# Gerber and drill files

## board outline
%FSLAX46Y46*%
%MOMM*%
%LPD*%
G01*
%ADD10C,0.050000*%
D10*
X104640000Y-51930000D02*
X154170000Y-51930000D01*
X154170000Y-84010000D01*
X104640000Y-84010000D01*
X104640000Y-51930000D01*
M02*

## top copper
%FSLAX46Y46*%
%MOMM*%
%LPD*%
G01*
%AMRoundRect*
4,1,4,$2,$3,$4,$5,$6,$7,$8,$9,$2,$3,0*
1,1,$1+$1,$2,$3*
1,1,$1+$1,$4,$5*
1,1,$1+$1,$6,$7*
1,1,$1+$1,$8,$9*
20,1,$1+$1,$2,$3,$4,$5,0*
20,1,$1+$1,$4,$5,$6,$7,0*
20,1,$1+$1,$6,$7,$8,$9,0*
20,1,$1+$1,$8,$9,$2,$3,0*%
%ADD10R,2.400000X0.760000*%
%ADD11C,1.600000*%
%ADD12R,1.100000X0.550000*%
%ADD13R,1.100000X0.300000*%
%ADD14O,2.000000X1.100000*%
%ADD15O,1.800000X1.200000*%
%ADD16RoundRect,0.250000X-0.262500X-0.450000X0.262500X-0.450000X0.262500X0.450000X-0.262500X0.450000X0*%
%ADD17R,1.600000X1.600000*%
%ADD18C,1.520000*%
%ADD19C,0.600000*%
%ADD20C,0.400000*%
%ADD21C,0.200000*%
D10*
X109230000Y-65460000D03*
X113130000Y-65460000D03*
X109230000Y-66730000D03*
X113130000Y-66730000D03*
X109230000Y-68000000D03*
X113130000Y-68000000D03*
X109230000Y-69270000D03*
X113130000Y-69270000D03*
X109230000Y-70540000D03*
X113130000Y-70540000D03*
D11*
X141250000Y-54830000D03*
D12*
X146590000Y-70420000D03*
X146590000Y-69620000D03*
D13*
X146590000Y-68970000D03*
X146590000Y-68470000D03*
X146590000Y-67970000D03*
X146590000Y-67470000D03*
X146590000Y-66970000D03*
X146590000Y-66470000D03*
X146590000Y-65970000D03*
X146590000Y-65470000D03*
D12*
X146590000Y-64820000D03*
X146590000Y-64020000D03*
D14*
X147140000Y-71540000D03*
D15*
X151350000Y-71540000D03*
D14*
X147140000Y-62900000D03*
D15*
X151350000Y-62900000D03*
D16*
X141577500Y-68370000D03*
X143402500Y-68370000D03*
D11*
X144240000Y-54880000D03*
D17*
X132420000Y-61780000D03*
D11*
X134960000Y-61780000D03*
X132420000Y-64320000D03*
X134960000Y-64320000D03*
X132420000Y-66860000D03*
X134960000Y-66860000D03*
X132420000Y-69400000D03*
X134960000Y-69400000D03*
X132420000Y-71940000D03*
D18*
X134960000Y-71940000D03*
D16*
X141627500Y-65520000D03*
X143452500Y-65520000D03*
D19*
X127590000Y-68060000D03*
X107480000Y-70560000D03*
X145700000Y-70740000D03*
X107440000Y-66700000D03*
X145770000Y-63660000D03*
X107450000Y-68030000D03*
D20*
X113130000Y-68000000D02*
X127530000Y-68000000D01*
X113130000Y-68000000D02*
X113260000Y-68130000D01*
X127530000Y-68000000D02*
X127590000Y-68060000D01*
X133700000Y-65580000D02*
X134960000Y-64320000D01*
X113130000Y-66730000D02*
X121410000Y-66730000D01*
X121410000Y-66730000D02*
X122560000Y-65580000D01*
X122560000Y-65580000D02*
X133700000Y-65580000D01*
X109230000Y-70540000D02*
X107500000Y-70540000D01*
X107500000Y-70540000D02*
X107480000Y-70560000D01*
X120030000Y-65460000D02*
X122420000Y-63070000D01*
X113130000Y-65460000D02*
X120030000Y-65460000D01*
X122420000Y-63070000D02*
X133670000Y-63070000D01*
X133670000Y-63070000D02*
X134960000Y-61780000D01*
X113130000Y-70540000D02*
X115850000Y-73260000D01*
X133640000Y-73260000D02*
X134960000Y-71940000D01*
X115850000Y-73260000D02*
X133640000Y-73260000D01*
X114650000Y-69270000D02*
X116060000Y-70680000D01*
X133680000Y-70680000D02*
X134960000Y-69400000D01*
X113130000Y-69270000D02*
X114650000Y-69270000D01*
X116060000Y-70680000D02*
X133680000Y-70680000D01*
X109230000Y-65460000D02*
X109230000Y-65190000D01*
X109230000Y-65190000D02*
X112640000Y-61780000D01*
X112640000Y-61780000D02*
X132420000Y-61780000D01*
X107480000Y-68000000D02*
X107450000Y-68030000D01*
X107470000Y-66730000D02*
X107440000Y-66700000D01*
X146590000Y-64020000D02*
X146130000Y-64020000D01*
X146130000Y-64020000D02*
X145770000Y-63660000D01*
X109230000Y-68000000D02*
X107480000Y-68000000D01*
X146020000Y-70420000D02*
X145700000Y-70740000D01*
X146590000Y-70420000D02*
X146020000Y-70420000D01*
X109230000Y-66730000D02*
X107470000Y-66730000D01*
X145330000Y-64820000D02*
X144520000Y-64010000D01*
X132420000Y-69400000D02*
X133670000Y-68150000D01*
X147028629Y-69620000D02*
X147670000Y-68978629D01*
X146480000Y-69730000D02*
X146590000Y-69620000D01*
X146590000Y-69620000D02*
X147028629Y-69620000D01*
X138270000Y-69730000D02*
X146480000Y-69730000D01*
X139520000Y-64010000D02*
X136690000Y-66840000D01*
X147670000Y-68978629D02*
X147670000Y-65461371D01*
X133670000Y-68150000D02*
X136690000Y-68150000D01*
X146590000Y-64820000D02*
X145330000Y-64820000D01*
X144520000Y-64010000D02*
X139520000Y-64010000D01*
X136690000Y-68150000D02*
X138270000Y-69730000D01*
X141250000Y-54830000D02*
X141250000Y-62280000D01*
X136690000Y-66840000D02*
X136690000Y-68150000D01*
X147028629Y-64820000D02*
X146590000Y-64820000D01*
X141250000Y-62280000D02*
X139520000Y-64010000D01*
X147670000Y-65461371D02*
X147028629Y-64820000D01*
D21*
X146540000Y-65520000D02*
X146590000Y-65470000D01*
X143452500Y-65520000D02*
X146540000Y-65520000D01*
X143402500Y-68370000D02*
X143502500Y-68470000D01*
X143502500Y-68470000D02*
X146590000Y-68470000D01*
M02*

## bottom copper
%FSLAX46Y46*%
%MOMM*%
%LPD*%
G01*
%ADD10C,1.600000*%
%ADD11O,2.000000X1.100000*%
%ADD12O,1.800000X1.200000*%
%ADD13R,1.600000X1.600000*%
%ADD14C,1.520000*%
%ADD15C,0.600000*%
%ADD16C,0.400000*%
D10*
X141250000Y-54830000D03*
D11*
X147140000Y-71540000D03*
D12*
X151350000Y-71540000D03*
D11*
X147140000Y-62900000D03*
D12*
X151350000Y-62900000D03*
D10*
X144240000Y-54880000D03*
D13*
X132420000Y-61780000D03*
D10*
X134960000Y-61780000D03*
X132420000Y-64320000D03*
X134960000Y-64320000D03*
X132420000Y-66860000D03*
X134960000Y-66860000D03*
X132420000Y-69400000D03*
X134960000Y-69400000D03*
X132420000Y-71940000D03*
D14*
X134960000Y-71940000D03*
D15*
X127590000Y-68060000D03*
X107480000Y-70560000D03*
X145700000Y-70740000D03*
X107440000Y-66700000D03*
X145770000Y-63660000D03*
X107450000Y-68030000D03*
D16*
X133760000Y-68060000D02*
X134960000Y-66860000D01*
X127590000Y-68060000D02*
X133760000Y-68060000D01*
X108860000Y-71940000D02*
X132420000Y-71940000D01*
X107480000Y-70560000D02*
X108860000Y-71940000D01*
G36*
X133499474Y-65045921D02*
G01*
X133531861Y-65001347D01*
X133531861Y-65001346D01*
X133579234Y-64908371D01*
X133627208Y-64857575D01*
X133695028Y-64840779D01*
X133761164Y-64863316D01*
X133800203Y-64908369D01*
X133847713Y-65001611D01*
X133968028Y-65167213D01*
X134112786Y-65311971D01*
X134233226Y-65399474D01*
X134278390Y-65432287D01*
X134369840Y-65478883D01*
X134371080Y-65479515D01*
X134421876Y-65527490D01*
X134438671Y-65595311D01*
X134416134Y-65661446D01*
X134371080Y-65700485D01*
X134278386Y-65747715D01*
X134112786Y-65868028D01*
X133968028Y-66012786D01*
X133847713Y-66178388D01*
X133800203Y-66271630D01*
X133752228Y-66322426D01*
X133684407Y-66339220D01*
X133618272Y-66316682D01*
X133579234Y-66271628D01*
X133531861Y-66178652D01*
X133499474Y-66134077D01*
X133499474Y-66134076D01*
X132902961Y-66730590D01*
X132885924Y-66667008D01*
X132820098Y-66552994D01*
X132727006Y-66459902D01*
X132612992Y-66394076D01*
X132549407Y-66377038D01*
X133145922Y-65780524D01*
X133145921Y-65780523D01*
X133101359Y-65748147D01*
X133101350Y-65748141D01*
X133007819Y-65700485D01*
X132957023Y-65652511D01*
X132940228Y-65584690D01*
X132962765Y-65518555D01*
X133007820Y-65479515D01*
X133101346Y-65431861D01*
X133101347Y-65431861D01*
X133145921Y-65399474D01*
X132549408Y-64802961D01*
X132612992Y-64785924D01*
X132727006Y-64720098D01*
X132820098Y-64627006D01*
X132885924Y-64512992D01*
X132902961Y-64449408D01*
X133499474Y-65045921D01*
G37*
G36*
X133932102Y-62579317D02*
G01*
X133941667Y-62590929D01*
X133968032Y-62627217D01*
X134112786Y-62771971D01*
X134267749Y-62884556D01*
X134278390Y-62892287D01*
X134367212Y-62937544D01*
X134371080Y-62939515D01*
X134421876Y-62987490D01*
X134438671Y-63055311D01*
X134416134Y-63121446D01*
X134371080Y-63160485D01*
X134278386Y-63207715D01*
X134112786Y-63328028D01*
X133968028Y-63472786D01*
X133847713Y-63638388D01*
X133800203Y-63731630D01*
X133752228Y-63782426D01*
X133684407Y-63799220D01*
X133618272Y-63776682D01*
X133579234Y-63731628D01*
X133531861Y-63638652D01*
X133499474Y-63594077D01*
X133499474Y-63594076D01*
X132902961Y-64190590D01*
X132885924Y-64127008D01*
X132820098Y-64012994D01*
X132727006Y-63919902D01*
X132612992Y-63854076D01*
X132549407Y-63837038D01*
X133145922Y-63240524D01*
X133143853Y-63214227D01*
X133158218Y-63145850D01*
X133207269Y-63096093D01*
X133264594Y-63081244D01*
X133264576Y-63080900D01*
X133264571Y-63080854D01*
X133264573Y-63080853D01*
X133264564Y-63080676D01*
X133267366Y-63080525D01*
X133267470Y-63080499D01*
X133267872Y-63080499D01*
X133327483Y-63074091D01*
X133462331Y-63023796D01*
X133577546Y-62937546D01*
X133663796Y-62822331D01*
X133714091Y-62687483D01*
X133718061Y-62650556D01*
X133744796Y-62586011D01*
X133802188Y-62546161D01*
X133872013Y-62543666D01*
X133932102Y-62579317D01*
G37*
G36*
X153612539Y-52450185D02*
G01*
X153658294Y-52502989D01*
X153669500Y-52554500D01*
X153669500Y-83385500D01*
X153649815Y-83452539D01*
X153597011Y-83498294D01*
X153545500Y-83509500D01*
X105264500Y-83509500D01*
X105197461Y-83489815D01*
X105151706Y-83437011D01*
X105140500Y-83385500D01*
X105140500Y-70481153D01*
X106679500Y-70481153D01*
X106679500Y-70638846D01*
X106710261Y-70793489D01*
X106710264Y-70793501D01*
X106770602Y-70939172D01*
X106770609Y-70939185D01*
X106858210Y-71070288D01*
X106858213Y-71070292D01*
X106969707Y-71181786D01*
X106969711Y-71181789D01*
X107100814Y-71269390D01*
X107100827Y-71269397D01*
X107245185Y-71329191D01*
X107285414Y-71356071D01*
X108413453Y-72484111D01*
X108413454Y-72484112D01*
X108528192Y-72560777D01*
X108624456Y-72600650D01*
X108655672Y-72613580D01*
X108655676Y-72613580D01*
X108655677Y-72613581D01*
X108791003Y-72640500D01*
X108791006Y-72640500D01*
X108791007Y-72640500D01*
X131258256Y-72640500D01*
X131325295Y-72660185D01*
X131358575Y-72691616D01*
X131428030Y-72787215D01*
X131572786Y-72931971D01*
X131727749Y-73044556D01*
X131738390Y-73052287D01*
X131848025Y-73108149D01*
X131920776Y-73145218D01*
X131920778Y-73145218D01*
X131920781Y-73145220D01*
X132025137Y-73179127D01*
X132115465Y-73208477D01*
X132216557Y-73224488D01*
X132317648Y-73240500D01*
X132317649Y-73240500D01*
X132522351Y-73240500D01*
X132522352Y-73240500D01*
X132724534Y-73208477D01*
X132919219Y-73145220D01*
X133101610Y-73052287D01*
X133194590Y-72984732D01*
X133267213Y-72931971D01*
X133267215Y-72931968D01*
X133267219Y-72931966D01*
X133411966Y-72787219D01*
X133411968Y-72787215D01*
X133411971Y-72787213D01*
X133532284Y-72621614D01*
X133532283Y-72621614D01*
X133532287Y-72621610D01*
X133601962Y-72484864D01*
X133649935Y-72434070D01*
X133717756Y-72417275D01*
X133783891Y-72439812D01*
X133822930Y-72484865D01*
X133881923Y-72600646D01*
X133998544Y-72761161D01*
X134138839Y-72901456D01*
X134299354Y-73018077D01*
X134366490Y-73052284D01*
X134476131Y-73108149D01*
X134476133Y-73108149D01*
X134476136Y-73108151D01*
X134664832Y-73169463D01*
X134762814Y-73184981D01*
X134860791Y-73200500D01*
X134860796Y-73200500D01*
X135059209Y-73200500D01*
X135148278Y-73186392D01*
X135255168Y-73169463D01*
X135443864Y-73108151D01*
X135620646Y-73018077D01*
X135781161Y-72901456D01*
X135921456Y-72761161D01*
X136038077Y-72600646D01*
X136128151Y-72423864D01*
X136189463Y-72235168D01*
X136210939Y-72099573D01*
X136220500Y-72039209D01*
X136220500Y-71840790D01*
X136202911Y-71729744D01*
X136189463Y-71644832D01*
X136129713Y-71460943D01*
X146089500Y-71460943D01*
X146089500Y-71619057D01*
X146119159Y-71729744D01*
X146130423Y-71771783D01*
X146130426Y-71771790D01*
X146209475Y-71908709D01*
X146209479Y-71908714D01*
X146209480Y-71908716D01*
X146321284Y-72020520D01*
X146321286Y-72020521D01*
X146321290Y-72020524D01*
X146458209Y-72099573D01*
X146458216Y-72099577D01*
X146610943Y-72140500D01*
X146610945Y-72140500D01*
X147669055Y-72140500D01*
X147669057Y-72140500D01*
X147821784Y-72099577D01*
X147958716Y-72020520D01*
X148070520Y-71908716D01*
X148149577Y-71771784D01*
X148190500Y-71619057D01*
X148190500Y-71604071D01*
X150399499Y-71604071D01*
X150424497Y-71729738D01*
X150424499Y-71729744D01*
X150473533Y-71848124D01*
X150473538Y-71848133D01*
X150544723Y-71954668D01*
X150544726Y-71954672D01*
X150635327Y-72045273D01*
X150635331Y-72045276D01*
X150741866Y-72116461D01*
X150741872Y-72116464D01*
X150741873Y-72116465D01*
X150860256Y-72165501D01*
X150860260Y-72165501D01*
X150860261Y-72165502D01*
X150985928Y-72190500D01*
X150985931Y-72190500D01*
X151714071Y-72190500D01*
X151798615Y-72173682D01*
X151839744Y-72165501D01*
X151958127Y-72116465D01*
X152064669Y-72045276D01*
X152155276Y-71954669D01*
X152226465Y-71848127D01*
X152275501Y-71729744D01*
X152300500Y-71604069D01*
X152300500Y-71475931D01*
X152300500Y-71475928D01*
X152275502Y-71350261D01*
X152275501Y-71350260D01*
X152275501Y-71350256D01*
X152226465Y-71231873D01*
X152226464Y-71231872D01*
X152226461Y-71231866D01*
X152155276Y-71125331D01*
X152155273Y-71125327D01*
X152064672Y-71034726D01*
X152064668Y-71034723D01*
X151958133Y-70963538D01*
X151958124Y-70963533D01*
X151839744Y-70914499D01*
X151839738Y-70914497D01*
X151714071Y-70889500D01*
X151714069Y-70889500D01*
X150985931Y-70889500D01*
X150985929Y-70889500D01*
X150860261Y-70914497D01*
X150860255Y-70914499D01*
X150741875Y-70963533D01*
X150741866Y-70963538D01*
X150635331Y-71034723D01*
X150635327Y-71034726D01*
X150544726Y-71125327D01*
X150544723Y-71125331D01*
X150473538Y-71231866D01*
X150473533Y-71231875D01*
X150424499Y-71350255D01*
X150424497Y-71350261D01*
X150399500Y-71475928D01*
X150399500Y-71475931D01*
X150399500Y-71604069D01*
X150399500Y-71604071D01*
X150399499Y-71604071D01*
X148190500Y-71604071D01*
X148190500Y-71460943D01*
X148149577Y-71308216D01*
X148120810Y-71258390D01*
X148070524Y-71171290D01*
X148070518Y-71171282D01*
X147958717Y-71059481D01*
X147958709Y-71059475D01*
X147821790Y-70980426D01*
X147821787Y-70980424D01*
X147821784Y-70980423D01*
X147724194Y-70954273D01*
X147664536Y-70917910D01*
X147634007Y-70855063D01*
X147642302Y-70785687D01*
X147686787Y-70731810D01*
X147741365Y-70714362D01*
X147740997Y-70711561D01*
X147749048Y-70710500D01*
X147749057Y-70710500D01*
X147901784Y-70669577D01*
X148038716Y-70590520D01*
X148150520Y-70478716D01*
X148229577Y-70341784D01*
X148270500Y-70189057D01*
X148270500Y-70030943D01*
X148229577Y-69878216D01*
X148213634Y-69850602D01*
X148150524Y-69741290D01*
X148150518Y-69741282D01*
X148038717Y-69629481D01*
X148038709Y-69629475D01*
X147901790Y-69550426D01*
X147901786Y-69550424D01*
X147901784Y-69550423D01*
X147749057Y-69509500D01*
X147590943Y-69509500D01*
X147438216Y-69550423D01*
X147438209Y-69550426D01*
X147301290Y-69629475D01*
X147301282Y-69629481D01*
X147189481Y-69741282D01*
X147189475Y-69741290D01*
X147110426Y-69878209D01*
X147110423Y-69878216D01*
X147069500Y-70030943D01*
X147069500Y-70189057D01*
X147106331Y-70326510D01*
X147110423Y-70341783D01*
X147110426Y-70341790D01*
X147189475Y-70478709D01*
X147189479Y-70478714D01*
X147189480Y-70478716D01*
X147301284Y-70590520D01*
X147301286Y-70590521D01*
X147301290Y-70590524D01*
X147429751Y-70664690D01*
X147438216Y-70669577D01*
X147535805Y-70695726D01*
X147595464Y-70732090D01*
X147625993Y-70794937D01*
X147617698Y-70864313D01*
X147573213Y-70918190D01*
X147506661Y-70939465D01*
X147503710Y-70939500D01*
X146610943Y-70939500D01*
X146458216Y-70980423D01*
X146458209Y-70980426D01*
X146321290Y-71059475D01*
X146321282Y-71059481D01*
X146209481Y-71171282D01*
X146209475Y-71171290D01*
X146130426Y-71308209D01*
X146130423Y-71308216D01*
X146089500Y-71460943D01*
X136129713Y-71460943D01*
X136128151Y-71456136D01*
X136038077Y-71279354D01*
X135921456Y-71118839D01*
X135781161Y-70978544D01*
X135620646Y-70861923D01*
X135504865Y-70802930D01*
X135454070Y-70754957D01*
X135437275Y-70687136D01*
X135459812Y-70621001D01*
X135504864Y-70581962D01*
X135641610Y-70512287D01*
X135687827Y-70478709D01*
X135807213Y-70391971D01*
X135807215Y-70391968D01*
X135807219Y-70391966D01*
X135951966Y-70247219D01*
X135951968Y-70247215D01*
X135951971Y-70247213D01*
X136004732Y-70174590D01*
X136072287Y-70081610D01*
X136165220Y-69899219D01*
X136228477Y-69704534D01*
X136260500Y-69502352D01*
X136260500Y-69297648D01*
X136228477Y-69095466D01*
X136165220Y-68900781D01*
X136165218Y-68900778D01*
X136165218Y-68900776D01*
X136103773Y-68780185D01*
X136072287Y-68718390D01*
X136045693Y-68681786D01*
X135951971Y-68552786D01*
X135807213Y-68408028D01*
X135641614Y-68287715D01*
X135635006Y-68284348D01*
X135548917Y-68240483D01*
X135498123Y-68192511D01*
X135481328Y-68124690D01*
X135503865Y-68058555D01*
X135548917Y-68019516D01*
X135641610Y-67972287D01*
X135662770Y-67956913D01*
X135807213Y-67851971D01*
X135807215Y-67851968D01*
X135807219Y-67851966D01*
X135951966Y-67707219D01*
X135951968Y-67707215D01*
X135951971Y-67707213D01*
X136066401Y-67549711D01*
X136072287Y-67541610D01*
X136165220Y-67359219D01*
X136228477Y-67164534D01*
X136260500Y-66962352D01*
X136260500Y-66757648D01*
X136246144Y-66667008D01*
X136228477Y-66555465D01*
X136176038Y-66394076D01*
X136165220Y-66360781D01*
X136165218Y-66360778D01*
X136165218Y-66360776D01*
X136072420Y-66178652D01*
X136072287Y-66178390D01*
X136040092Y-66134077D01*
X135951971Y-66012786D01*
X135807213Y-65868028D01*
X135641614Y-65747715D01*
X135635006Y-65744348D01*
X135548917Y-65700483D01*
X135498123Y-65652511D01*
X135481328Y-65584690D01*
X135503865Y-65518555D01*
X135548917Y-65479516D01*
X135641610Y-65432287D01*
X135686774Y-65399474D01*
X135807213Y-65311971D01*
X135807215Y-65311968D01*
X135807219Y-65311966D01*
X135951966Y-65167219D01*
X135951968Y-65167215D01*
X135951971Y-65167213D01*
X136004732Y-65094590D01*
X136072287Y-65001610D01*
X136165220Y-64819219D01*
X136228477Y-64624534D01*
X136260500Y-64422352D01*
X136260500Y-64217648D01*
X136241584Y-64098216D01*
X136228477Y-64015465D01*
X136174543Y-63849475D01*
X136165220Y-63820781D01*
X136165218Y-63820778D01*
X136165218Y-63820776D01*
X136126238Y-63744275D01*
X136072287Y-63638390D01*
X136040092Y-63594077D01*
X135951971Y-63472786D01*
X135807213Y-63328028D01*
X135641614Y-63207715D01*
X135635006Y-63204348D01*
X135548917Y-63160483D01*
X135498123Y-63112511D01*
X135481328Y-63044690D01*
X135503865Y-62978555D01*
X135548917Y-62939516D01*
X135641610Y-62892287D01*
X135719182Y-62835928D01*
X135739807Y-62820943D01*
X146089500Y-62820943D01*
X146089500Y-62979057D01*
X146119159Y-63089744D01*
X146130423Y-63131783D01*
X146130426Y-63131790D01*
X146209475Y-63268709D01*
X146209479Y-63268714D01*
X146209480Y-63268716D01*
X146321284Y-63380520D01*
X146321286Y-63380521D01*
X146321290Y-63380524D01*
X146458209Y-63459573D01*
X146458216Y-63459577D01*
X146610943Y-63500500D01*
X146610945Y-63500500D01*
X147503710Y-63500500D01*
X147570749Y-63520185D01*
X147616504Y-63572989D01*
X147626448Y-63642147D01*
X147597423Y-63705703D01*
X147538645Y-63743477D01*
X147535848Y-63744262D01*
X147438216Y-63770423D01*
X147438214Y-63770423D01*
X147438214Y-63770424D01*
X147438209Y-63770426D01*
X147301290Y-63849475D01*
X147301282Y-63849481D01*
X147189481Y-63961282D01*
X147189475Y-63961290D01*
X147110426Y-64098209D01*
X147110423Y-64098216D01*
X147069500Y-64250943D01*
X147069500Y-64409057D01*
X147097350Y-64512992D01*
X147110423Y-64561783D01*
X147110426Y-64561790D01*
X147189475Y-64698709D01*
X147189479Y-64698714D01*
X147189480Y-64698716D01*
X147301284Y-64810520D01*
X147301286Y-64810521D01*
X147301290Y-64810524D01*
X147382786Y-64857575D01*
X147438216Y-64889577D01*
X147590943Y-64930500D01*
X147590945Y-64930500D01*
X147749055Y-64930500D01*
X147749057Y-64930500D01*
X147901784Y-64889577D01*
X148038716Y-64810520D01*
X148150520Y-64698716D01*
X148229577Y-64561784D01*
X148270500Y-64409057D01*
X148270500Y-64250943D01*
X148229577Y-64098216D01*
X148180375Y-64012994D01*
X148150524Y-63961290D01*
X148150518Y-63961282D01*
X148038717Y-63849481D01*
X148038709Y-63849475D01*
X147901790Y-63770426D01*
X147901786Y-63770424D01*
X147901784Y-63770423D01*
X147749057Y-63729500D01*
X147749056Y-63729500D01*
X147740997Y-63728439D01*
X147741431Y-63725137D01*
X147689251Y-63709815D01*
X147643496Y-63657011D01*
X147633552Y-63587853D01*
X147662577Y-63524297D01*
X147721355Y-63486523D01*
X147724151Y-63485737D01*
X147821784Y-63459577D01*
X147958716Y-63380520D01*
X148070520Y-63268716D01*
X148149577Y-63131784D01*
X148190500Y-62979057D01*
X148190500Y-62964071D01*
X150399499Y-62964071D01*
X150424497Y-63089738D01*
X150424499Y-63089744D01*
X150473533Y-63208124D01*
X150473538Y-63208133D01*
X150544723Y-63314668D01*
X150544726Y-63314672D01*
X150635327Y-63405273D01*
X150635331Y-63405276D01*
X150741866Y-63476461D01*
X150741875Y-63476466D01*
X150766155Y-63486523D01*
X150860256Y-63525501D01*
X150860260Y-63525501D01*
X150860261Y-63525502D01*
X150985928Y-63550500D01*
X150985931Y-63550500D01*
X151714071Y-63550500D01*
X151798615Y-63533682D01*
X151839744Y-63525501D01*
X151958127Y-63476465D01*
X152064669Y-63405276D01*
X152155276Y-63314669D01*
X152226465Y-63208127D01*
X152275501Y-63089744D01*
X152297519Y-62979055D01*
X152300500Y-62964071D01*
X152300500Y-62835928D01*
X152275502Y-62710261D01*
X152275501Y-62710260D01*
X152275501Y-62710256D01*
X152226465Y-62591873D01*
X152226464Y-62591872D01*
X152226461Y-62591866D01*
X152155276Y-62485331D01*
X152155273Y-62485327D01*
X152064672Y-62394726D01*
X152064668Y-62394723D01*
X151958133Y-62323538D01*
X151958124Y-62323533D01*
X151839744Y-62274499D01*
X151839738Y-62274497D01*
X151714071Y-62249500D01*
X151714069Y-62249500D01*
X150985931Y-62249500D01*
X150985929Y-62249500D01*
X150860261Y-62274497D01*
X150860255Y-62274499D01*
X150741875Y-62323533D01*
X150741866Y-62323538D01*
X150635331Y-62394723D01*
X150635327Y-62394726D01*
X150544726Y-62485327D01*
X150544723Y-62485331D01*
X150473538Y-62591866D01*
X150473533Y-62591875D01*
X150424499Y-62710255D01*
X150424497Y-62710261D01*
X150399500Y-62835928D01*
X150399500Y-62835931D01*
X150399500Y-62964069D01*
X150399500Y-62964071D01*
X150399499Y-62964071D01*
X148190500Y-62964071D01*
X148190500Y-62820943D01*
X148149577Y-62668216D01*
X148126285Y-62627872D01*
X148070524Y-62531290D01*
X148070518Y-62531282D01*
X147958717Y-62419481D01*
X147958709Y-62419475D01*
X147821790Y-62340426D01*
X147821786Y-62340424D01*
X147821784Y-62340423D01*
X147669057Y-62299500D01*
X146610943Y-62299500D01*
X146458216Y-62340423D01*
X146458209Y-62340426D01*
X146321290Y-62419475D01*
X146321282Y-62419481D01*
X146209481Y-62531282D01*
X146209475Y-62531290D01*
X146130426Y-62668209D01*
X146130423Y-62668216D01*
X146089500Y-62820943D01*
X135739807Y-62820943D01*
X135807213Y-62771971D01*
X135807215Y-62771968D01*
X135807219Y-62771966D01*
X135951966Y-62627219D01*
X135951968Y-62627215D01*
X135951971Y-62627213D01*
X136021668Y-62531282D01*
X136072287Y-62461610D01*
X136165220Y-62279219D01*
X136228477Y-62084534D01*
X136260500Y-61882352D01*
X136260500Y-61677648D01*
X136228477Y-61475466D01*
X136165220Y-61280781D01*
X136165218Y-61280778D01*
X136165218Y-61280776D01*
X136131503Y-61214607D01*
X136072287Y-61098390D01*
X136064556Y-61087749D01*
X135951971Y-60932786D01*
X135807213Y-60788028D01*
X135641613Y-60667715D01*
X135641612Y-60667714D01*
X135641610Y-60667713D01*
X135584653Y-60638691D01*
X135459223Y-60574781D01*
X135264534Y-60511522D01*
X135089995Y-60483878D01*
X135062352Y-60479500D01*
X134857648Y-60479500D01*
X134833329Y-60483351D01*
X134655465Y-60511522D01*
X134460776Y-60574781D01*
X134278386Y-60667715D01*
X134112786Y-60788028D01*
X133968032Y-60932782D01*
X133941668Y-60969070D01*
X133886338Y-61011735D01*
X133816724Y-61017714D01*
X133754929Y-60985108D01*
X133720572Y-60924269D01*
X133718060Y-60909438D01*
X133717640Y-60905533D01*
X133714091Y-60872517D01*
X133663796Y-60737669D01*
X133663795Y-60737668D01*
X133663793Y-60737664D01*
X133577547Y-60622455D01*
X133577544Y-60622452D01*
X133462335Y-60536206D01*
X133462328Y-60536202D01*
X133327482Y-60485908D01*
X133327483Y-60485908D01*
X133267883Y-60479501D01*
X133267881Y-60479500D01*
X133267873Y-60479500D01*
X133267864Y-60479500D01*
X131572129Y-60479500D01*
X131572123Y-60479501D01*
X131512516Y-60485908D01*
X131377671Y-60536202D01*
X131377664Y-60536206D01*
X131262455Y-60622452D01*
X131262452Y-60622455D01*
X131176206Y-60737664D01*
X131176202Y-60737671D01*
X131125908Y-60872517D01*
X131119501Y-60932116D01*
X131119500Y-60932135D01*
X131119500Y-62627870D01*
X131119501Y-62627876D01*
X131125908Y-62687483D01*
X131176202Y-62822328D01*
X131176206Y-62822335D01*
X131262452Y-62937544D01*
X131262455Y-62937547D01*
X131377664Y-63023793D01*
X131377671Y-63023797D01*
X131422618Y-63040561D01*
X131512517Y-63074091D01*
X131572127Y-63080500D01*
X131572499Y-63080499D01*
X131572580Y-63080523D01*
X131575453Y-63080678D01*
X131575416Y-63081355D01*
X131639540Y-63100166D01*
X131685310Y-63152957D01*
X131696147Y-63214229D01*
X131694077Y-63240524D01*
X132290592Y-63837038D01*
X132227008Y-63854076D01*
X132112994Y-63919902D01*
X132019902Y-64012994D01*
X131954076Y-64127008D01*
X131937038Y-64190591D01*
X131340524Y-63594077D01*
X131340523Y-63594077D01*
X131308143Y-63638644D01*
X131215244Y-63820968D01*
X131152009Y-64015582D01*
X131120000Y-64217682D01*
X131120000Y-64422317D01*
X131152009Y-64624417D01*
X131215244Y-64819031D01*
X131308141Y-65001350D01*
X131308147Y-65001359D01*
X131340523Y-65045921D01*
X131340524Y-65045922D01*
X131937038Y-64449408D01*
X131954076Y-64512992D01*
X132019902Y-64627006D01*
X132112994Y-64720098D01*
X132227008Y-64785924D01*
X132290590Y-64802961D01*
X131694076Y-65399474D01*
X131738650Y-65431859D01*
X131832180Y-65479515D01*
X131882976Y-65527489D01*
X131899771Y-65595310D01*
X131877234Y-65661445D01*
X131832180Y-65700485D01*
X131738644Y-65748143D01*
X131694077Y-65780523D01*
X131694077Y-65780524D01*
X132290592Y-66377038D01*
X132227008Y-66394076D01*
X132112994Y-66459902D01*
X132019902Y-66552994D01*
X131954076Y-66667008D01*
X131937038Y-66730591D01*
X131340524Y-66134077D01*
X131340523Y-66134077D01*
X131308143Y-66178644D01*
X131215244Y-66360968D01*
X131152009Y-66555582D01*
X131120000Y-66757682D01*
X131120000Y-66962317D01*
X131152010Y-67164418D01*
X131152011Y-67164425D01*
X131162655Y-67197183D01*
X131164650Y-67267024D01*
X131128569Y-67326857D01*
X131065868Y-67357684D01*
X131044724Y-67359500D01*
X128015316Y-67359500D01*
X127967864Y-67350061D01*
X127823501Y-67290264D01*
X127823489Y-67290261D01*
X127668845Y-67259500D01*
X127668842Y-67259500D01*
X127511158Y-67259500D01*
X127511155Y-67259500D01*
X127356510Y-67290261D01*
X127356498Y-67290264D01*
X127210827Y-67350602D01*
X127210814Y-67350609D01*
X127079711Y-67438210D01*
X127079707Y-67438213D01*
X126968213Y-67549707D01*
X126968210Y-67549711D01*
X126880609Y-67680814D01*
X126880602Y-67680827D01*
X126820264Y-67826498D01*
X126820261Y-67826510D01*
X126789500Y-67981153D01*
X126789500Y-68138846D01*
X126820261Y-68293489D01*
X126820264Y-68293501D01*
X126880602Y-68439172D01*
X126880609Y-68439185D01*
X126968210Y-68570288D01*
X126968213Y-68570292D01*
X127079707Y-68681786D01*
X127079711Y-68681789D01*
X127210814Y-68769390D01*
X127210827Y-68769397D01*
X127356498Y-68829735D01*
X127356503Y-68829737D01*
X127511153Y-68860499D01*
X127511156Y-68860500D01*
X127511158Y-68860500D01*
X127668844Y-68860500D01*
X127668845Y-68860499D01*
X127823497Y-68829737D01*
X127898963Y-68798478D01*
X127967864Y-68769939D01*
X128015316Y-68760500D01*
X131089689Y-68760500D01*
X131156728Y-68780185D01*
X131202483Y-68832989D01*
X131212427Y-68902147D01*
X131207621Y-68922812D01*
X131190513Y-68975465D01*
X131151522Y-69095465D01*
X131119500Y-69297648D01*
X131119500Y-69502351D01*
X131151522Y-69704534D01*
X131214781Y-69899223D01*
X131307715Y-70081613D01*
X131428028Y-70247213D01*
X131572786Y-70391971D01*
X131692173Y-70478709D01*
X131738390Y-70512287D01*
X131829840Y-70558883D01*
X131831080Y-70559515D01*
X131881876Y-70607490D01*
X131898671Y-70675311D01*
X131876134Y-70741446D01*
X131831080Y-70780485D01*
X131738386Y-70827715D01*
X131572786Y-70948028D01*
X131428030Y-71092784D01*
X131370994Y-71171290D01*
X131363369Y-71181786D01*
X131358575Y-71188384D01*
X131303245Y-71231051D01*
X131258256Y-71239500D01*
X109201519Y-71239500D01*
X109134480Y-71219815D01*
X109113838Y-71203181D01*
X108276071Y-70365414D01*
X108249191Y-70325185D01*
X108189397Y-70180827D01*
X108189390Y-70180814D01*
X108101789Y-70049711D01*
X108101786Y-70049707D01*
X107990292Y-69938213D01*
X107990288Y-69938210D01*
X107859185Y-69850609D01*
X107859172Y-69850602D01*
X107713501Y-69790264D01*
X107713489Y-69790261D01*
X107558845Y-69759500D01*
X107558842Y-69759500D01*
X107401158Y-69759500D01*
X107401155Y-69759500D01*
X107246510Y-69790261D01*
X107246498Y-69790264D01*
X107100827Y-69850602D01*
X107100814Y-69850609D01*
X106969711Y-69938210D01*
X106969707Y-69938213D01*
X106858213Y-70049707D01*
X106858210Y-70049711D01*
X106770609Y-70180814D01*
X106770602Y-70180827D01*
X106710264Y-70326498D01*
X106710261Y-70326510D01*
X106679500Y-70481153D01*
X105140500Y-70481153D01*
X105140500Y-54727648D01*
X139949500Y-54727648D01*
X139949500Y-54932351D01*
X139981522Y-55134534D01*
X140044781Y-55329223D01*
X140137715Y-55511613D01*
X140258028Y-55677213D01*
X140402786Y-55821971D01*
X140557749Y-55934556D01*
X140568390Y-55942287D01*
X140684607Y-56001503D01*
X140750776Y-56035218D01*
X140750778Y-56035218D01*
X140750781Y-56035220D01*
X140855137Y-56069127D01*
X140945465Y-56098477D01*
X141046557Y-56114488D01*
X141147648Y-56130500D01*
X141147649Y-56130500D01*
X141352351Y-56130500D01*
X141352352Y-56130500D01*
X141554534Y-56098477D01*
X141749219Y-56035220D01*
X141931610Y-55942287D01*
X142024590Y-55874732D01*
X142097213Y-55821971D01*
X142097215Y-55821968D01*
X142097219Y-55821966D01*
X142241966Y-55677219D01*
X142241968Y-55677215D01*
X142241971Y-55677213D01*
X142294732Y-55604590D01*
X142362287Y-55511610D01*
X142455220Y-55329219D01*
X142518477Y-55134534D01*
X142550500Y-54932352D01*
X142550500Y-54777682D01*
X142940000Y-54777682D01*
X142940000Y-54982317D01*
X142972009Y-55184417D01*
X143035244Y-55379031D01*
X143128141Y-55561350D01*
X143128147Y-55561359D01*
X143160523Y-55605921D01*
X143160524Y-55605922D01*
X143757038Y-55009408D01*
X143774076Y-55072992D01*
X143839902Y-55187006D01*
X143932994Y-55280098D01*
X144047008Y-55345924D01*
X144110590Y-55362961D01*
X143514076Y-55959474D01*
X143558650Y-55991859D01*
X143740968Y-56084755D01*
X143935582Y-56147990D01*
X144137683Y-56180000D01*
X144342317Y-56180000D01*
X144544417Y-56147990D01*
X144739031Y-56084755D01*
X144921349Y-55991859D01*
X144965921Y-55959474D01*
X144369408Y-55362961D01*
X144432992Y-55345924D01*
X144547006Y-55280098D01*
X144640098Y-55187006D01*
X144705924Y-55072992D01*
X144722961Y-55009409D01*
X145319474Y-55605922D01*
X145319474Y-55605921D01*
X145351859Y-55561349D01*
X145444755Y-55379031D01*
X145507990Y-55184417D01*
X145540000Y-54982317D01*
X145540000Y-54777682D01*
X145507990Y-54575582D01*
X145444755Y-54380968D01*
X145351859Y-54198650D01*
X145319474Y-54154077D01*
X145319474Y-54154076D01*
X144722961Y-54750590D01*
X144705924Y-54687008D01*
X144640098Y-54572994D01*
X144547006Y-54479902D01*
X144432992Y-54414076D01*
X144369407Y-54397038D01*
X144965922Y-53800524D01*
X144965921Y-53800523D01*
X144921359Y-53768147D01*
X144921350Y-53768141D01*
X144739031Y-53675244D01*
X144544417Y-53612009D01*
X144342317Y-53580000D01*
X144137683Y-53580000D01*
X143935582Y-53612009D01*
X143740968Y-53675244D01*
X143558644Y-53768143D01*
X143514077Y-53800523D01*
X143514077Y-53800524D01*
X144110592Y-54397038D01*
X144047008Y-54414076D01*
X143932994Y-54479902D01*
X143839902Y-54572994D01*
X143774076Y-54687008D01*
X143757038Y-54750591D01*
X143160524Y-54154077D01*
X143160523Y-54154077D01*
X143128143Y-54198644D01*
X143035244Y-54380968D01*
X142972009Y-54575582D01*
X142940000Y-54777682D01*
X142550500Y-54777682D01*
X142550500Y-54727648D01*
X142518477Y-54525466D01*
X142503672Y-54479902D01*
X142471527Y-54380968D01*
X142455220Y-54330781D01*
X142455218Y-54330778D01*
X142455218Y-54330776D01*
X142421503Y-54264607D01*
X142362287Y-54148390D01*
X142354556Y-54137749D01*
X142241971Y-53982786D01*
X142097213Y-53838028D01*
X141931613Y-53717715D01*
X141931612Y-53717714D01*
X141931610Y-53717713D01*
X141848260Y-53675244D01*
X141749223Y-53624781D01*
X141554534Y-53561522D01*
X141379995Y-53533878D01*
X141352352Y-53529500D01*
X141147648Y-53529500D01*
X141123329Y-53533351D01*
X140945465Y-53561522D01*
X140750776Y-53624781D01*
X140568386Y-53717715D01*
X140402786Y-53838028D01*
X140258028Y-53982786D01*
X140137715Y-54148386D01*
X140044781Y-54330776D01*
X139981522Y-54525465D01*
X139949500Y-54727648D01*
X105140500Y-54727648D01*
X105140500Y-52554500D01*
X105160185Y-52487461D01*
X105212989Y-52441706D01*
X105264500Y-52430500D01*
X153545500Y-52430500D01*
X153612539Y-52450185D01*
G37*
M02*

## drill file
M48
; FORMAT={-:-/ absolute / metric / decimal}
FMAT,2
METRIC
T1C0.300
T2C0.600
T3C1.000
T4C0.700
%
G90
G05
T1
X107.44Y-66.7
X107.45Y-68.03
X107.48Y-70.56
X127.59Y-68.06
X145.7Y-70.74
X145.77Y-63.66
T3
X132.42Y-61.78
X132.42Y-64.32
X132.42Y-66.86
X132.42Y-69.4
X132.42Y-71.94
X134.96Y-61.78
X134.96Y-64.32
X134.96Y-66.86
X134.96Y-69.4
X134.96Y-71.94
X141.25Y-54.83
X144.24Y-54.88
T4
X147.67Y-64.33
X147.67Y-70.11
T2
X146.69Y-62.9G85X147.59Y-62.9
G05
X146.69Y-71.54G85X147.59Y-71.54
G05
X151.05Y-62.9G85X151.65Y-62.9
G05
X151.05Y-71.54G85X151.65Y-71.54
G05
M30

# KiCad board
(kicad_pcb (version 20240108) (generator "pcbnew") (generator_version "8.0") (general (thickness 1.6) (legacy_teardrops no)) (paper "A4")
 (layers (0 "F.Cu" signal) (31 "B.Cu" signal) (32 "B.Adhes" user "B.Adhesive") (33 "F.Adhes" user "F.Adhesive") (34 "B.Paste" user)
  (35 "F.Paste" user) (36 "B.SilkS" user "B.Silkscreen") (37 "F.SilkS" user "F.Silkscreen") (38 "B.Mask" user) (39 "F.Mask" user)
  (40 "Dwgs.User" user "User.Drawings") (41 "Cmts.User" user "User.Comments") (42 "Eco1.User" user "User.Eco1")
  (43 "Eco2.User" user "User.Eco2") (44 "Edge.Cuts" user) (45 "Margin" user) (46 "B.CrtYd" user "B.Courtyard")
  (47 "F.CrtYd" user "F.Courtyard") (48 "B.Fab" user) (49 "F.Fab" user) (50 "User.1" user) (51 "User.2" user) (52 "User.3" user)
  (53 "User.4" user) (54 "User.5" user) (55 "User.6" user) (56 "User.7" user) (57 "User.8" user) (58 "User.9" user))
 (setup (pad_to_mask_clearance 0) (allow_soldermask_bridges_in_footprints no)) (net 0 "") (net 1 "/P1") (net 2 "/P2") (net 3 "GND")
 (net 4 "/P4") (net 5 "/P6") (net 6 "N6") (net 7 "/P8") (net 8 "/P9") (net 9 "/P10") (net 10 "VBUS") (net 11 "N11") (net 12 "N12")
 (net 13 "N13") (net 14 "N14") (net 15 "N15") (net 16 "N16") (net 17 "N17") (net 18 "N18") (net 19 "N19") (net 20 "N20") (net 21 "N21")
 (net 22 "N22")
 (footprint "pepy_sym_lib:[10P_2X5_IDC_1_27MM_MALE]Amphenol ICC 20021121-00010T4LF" (layer "F.Cu") (at 111.18 68 -90)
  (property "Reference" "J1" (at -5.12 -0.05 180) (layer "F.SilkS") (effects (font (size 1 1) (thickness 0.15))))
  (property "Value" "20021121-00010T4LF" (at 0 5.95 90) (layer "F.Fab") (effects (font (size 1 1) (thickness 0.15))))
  (pad "1" smd rect (at -2.54 1.95 270) (size 0.76 2.4) (layers "F.Cu" "F.Paste" "F.Mask") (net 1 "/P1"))
  (pad "2" smd rect (at -2.54 -1.95 270) (size 0.76 2.4) (layers "F.Cu" "F.Paste" "F.Mask") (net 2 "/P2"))
  (pad "3" smd rect (at -1.27 1.95 270) (size 0.76 2.4) (layers "F.Cu" "F.Paste" "F.Mask") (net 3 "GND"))
  (pad "4" smd rect (at -1.27 -1.95 270) (size 0.76 2.4) (layers "F.Cu" "F.Paste" "F.Mask") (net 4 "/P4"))
  (pad "5" smd rect (at 0 1.95 270) (size 0.76 2.4) (layers "F.Cu" "F.Paste" "F.Mask") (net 3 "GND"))
  (pad "6" smd rect (at 0 -1.95 270) (size 0.76 2.4) (layers "F.Cu" "F.Paste" "F.Mask") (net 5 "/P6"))
  (pad "7" smd rect (at 1.27 1.95 270) (size 0.76 2.4) (layers "F.Cu" "F.Paste" "F.Mask") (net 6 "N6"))
  (pad "8" smd rect (at 1.27 -1.95 270) (size 0.76 2.4) (layers "F.Cu" "F.Paste" "F.Mask") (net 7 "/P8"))
  (pad "9" smd rect (at 2.54 1.95 270) (size 0.76 2.4) (layers "F.Cu" "F.Paste" "F.Mask") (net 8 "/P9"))
  (pad "10" smd rect (at 2.54 -1.95 270) (size 0.76 2.4) (layers "F.Cu" "F.Paste" "F.Mask") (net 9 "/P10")))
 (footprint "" (layer "F.Cu") (at 141.25 54.83)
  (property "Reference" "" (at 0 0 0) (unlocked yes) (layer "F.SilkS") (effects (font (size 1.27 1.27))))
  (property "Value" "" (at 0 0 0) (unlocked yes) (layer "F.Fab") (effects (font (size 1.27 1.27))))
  (pad "7" thru_hole circle (at 0 0 90) (size 1.6 1.6) (drill 0.999998) (layers "*.Cu" "*.Mask") (remove_unused_layers no) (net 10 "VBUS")))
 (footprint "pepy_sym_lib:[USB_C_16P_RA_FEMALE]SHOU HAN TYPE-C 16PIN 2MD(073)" (layer "F.Cu") (at 148.97 67.22 90)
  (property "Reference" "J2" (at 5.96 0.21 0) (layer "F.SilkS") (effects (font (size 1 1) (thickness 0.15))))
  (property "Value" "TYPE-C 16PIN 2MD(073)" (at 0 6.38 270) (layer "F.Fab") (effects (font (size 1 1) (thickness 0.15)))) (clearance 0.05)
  (pad "" np_thru_hole circle (at -2.89 -1.3 90) (size 0.7 0.7) (drill 0.7) (layers "F&B.Cu" "*.Mask"))
  (pad "" np_thru_hole circle (at 2.89 -1.3 90) (size 0.7 0.7) (drill 0.7) (layers "F&B.Cu" "*.Mask"))
  (pad "1" smd rect (at -3.2 -2.38 90) (size 0.55 1.1) (layers "F.Cu" "F.Paste" "F.Mask") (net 3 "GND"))
  (pad "2" smd rect (at -2.4 -2.38 90) (size 0.55 1.1) (layers "F.Cu" "F.Paste" "F.Mask") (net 10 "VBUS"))
  (pad "3" smd rect (at -1.75 -2.38 90) (size 0.3 1.1) (layers "F.Cu" "F.Paste" "F.Mask") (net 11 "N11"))
  (pad "4" smd rect (at -1.25 -2.38 90) (size 0.3 1.1) (layers "F.Cu" "F.Paste" "F.Mask") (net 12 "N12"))
  (pad "5" smd rect (at -0.75 -2.38 90) (size 0.3 1.1) (layers "F.Cu" "F.Paste" "F.Mask") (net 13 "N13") (clearance 0.05))
  (pad "6" smd rect (at -0.25 -2.38 90) (size 0.3 1.1) (layers "F.Cu" "F.Paste" "F.Mask") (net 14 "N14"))
  (pad "7" smd rect (at 0.25 -2.38 90) (size 0.3 1.1) (layers "F.Cu" "F.Paste" "F.Mask") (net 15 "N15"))
  (pad "8" smd rect (at 0.75 -2.38 90) (size 0.3 1.1) (layers "F.Cu" "F.Paste" "F.Mask") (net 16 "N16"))
  (pad "9" smd rect (at 1.25 -2.38 90) (size 0.3 1.1) (layers "F.Cu" "F.Paste" "F.Mask") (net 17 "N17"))
  (pad "10" smd rect (at 1.75 -2.38 90) (size 0.3 1.1) (layers "F.Cu" "F.Paste" "F.Mask") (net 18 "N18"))
  (pad "11" smd rect (at 2.4 -2.38 90) (size 0.55 1.1) (layers "F.Cu" "F.Paste" "F.Mask") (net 10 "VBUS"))
  (pad "12" smd rect (at 3.2 -2.38 90) (size 0.55 1.1) (layers "F.Cu" "F.Paste" "F.Mask") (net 3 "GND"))
  (pad "13" thru_hole oval (at -4.32 -1.83 90) (size 1.1 2) (drill oval 0.599999 1.499997) (layers "*.Cu" "*.Mask")
   (remove_unused_layers no) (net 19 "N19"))
  (pad "13" thru_hole oval (at -4.32 2.38 90) (size 1.2 1.8) (drill oval 0.599999 1.199998) (layers "*.Cu" "*.Mask")
   (remove_unused_layers no) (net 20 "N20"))
  (pad "14" thru_hole oval (at 4.32 -1.83 90) (size 1.1 2) (drill oval 0.599999 1.500022) (layers "*.Cu" "*.Mask") (remove_unused_layers no)
   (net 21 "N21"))
  (pad "14" thru_hole oval (at 4.32 2.38 90) (size 1.2 1.8) (drill oval 0.599999 1.199998) (layers "*.Cu" "*.Mask")
   (remove_unused_layers no) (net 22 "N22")))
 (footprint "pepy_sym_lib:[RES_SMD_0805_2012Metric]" (layer "F.Cu") (at 142.49 68.37)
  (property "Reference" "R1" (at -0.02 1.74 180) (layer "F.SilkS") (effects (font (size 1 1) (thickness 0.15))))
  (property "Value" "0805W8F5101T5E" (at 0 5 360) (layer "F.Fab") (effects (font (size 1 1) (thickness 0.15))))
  (pad "1" smd roundrect (at -0.9125 0) (size 1.025 1.4) (layers "F.Cu" "F.Paste" "F.Mask") (roundrect_rratio 0.243902) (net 3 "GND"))
  (pad "2" smd roundrect (at 0.9125 0) (size 1.025 1.4) (layers "F.Cu" "F.Paste" "F.Mask") (roundrect_rratio 0.243902) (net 12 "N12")))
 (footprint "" (layer "F.Cu") (at 144.24 54.88)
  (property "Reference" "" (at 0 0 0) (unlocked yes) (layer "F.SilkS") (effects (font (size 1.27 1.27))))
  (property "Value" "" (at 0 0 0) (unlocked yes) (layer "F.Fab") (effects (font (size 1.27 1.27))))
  (pad "3" thru_hole circle (at 0 0 90) (size 1.6 1.6) (drill 0.999998) (layers "*.Cu" "*.Mask") (remove_unused_layers no) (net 3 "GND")))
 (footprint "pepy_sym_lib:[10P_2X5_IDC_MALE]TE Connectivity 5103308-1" (layer "F.Cu") (at 133.69 66.86 90)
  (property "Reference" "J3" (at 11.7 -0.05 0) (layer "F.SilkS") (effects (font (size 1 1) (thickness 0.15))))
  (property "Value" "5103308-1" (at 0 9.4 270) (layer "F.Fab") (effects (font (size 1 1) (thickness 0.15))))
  (pad "1" thru_hole rect (at 5.08 -1.27 90) (size 1.6 1.6) (drill 0.999998) (layers "*.Cu" "*.Mask") (remove_unused_layers no)
   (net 1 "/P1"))
  (pad "2" thru_hole circle (at 5.08 1.27 90) (size 1.6 1.6) (drill 0.999998) (layers "*.Cu" "*.Mask") (remove_unused_layers no)
   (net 2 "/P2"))
  (pad "3" thru_hole circle (at 2.54 -1.27 90) (size 1.6 1.6) (drill 0.999998) (layers "*.Cu" "*.Mask") (remove_unused_layers no)
   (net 3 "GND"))
  (pad "4" thru_hole circle (at 2.54 1.27 90) (size 1.6 1.6) (drill 0.999998) (layers "*.Cu" "*.Mask") (remove_unused_layers no)
   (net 4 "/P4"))
  (pad "5" thru_hole circle (at 0 -1.27 90) (size 1.6 1.6) (drill 0.999998) (layers "*.Cu" "*.Mask") (remove_unused_layers no) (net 3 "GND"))
  (pad "6" thru_hole circle (at 0 1.27 90) (size 1.6 1.6) (drill 0.999998) (layers "*.Cu" "*.Mask") (remove_unused_layers no) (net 5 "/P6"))
  (pad "7" thru_hole circle (at -2.54 -1.27 90) (size 1.6 1.6) (drill 0.999998) (layers "*.Cu" "*.Mask") (remove_unused_layers no)
   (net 10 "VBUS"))
  (pad "8" thru_hole circle (at -2.54 1.27 90) (size 1.6 1.6) (drill 0.999998) (layers "*.Cu" "*.Mask") (remove_unused_layers no)
   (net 7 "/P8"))
  (pad "9" thru_hole circle (at -5.08 -1.27 90) (size 1.6 1.6) (drill 0.999998) (layers "*.Cu" "*.Mask") (remove_unused_layers no)
   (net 8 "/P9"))
  (pad "10" thru_hole circle (at -5.08 1.27 90) (size 1.52 1.52) (drill 0.999998) (layers "*.Cu" "*.Mask") (remove_unused_layers no)
   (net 9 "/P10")))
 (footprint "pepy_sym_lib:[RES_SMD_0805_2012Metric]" (layer "F.Cu") (at 142.54 65.52)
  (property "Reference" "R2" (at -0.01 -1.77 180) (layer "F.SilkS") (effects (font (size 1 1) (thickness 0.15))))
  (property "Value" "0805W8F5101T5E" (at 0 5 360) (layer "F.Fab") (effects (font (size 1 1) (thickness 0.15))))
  (pad "1" smd roundrect (at -0.9125 0) (size 1.025 1.4) (layers "F.Cu" "F.Paste" "F.Mask") (roundrect_rratio 0.243902) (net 3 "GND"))
  (pad "2" smd roundrect (at 0.9125 0) (size 1.025 1.4) (layers "F.Cu" "F.Paste" "F.Mask") (roundrect_rratio 0.243902) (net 18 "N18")))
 (gr_rect (start 104.64 51.93) (end 154.17 84.01) (stroke (width 0.05) (type default)) (fill none) (layer "Edge.Cuts"))
 (segment (start 113.13 68) (end 127.53 68) (width 0.4) (layer "F.Cu") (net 5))
 (segment (start 113.13 68) (end 113.26 68.13) (width 0.4) (layer "F.Cu") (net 5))
 (segment (start 127.53 68) (end 127.59 68.06) (width 0.4) (layer "F.Cu") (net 5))
 (via (at 127.59 68.06) (size 0.6) (drill 0.3) (layers "F.Cu" "B.Cu") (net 5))
 (segment (start 133.76 68.06) (end 134.96 66.86) (width 0.4) (layer "B.Cu") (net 5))
 (segment (start 127.59 68.06) (end 133.76 68.06) (width 0.4) (layer "B.Cu") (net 5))
 (segment (start 133.7 65.58) (end 134.96 64.32) (width 0.4) (layer "F.Cu") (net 4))
 (segment (start 113.13 66.73) (end 121.41 66.73) (width 0.4) (layer "F.Cu") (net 4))
 (segment (start 121.41 66.73) (end 122.56 65.58) (width 0.4) (layer "F.Cu") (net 4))
 (segment (start 122.56 65.58) (end 133.7 65.58) (width 0.4) (layer "F.Cu") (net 4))
 (segment (start 109.23 70.54) (end 107.5 70.54) (width 0.4) (layer "F.Cu") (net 8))
 (segment (start 107.5 70.54) (end 107.48 70.56) (width 0.4) (layer "F.Cu") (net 8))
 (via (at 107.48 70.56) (size 0.6) (drill 0.3) (layers "F.Cu" "B.Cu") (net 8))
 (segment (start 108.86 71.94) (end 132.42 71.94) (width 0.4) (layer "B.Cu") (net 8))
 (segment (start 107.48 70.56) (end 108.86 71.94) (width 0.4) (layer "B.Cu") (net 8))
 (segment (start 120.03 65.46) (end 122.42 63.07) (width 0.4) (layer "F.Cu") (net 2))
 (segment (start 113.13 65.46) (end 120.03 65.46) (width 0.4) (layer "F.Cu") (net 2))
 (segment (start 122.42 63.07) (end 133.67 63.07) (width 0.4) (layer "F.Cu") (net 2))
 (segment (start 133.67 63.07) (end 134.96 61.78) (width 0.4) (layer "F.Cu") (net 2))
 (segment (start 113.13 70.54) (end 115.85 73.26) (width 0.4) (layer "F.Cu") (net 9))
 (segment (start 133.64 73.26) (end 134.96 71.94) (width 0.4) (layer "F.Cu") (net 9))
 (segment (start 115.85 73.26) (end 133.64 73.26) (width 0.4) (layer "F.Cu") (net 9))
 (segment (start 114.65 69.27) (end 116.06 70.68) (width 0.4) (layer "F.Cu") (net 7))
 (segment (start 133.68 70.68) (end 134.96 69.4) (width 0.4) (layer "F.Cu") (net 7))
 (segment (start 113.13 69.27) (end 114.65 69.27) (width 0.4) (layer "F.Cu") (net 7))
 (segment (start 116.06 70.68) (end 133.68 70.68) (width 0.4) (layer "F.Cu") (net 7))
 (segment (start 109.23 65.46) (end 109.23 65.19) (width 0.4) (layer "F.Cu") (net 1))
 (segment (start 109.23 65.19) (end 112.64 61.78) (width 0.4) (layer "F.Cu") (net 1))
 (segment (start 112.64 61.78) (end 132.42 61.78) (width 0.4) (layer "F.Cu") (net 1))
 (segment (start 107.48 68) (end 107.45 68.03) (width 0.4) (layer "F.Cu") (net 3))
 (segment (start 107.47 66.73) (end 107.44 66.7) (width 0.4) (layer "F.Cu") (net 3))
 (segment (start 146.59 64.02) (end 146.13 64.02) (width 0.4) (layer "F.Cu") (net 3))
 (segment (start 146.13 64.02) (end 145.77 63.66) (width 0.4) (layer "F.Cu") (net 3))
 (segment (start 109.23 68) (end 107.48 68) (width 0.4) (layer "F.Cu") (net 3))
 (segment (start 146.02 70.42) (end 145.7 70.74) (width 0.4) (layer "F.Cu") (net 3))
 (segment (start 146.59 70.42) (end 146.02 70.42) (width 0.4) (layer "F.Cu") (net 3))
 (segment (start 109.23 66.73) (end 107.47 66.73) (width 0.4) (layer "F.Cu") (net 3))
 (via (at 145.7 70.74) (size 0.6) (drill 0.3) (layers "F.Cu" "B.Cu") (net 3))
 (via (at 107.44 66.7) (size 0.6) (drill 0.3) (layers "F.Cu" "B.Cu") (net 3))
 (via (at 145.77 63.66) (size 0.6) (drill 0.3) (layers "F.Cu" "B.Cu") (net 3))
 (via (at 107.45 68.03) (size 0.6) (drill 0.3) (layers "F.Cu" "B.Cu") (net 3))
 (segment (start 145.33 64.82) (end 144.52 64.01) (width 0.4) (layer "F.Cu") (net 10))
 (segment (start 132.42 69.4) (end 133.67 68.15) (width 0.4) (layer "F.Cu") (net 10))
 (segment (start 147.028629 69.62) (end 147.67 68.978629) (width 0.4) (layer "F.Cu") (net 10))
 (segment (start 146.48 69.73) (end 146.59 69.62) (width 0.4) (layer "F.Cu") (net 10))
 (segment (start 146.59 69.62) (end 147.028629 69.62) (width 0.4) (layer "F.Cu") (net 10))
 (segment (start 138.27 69.73) (end 146.48 69.73) (width 0.4) (layer "F.Cu") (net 10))
 (segment (start 139.52 64.01) (end 136.69 66.84) (width 0.4) (layer "F.Cu") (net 10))
 (segment (start 147.67 68.978629) (end 147.67 65.461371) (width 0.4) (layer "F.Cu") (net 10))
 (segment (start 133.67 68.15) (end 136.69 68.15) (width 0.4) (layer "F.Cu") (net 10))
 (segment (start 146.59 64.82) (end 145.33 64.82) (width 0.4) (layer "F.Cu") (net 10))
 (segment (start 144.52 64.01) (end 139.52 64.01) (width 0.4) (layer "F.Cu") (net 10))
 (segment (start 136.69 68.15) (end 138.27 69.73) (width 0.4) (layer "F.Cu") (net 10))
 (segment (start 141.25 54.83) (end 141.25 62.28) (width 0.4) (layer "F.Cu") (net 10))
 (segment (start 136.69 66.84) (end 136.69 68.15) (width 0.4) (layer "F.Cu") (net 10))
 (segment (start 147.028629 64.82) (end 146.59 64.82) (width 0.4) (layer "F.Cu") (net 10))
 (segment (start 141.25 62.28) (end 139.52 64.01) (width 0.4) (layer "F.Cu") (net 10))
 (segment (start 147.67 65.461371) (end 147.028629 64.82) (width 0.4) (layer "F.Cu") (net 10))
 (segment (start 146.54 65.52) (end 146.59 65.47) (width 0.2) (layer "F.Cu") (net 18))
 (segment (start 143.4525 65.52) (end 146.54 65.52) (width 0.2) (layer "F.Cu") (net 18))
 (segment (start 143.4025 68.37) (end 143.5025 68.47) (width 0.2) (layer "F.Cu") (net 12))
 (segment (start 143.5025 68.47) (end 146.59 68.47) (width 0.2) (layer "F.Cu") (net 12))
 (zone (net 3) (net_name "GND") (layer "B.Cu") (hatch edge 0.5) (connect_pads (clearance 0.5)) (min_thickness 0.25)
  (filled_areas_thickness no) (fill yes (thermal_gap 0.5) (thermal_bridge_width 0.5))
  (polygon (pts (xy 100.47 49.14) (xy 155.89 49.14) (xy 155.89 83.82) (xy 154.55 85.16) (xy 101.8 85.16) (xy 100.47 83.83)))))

